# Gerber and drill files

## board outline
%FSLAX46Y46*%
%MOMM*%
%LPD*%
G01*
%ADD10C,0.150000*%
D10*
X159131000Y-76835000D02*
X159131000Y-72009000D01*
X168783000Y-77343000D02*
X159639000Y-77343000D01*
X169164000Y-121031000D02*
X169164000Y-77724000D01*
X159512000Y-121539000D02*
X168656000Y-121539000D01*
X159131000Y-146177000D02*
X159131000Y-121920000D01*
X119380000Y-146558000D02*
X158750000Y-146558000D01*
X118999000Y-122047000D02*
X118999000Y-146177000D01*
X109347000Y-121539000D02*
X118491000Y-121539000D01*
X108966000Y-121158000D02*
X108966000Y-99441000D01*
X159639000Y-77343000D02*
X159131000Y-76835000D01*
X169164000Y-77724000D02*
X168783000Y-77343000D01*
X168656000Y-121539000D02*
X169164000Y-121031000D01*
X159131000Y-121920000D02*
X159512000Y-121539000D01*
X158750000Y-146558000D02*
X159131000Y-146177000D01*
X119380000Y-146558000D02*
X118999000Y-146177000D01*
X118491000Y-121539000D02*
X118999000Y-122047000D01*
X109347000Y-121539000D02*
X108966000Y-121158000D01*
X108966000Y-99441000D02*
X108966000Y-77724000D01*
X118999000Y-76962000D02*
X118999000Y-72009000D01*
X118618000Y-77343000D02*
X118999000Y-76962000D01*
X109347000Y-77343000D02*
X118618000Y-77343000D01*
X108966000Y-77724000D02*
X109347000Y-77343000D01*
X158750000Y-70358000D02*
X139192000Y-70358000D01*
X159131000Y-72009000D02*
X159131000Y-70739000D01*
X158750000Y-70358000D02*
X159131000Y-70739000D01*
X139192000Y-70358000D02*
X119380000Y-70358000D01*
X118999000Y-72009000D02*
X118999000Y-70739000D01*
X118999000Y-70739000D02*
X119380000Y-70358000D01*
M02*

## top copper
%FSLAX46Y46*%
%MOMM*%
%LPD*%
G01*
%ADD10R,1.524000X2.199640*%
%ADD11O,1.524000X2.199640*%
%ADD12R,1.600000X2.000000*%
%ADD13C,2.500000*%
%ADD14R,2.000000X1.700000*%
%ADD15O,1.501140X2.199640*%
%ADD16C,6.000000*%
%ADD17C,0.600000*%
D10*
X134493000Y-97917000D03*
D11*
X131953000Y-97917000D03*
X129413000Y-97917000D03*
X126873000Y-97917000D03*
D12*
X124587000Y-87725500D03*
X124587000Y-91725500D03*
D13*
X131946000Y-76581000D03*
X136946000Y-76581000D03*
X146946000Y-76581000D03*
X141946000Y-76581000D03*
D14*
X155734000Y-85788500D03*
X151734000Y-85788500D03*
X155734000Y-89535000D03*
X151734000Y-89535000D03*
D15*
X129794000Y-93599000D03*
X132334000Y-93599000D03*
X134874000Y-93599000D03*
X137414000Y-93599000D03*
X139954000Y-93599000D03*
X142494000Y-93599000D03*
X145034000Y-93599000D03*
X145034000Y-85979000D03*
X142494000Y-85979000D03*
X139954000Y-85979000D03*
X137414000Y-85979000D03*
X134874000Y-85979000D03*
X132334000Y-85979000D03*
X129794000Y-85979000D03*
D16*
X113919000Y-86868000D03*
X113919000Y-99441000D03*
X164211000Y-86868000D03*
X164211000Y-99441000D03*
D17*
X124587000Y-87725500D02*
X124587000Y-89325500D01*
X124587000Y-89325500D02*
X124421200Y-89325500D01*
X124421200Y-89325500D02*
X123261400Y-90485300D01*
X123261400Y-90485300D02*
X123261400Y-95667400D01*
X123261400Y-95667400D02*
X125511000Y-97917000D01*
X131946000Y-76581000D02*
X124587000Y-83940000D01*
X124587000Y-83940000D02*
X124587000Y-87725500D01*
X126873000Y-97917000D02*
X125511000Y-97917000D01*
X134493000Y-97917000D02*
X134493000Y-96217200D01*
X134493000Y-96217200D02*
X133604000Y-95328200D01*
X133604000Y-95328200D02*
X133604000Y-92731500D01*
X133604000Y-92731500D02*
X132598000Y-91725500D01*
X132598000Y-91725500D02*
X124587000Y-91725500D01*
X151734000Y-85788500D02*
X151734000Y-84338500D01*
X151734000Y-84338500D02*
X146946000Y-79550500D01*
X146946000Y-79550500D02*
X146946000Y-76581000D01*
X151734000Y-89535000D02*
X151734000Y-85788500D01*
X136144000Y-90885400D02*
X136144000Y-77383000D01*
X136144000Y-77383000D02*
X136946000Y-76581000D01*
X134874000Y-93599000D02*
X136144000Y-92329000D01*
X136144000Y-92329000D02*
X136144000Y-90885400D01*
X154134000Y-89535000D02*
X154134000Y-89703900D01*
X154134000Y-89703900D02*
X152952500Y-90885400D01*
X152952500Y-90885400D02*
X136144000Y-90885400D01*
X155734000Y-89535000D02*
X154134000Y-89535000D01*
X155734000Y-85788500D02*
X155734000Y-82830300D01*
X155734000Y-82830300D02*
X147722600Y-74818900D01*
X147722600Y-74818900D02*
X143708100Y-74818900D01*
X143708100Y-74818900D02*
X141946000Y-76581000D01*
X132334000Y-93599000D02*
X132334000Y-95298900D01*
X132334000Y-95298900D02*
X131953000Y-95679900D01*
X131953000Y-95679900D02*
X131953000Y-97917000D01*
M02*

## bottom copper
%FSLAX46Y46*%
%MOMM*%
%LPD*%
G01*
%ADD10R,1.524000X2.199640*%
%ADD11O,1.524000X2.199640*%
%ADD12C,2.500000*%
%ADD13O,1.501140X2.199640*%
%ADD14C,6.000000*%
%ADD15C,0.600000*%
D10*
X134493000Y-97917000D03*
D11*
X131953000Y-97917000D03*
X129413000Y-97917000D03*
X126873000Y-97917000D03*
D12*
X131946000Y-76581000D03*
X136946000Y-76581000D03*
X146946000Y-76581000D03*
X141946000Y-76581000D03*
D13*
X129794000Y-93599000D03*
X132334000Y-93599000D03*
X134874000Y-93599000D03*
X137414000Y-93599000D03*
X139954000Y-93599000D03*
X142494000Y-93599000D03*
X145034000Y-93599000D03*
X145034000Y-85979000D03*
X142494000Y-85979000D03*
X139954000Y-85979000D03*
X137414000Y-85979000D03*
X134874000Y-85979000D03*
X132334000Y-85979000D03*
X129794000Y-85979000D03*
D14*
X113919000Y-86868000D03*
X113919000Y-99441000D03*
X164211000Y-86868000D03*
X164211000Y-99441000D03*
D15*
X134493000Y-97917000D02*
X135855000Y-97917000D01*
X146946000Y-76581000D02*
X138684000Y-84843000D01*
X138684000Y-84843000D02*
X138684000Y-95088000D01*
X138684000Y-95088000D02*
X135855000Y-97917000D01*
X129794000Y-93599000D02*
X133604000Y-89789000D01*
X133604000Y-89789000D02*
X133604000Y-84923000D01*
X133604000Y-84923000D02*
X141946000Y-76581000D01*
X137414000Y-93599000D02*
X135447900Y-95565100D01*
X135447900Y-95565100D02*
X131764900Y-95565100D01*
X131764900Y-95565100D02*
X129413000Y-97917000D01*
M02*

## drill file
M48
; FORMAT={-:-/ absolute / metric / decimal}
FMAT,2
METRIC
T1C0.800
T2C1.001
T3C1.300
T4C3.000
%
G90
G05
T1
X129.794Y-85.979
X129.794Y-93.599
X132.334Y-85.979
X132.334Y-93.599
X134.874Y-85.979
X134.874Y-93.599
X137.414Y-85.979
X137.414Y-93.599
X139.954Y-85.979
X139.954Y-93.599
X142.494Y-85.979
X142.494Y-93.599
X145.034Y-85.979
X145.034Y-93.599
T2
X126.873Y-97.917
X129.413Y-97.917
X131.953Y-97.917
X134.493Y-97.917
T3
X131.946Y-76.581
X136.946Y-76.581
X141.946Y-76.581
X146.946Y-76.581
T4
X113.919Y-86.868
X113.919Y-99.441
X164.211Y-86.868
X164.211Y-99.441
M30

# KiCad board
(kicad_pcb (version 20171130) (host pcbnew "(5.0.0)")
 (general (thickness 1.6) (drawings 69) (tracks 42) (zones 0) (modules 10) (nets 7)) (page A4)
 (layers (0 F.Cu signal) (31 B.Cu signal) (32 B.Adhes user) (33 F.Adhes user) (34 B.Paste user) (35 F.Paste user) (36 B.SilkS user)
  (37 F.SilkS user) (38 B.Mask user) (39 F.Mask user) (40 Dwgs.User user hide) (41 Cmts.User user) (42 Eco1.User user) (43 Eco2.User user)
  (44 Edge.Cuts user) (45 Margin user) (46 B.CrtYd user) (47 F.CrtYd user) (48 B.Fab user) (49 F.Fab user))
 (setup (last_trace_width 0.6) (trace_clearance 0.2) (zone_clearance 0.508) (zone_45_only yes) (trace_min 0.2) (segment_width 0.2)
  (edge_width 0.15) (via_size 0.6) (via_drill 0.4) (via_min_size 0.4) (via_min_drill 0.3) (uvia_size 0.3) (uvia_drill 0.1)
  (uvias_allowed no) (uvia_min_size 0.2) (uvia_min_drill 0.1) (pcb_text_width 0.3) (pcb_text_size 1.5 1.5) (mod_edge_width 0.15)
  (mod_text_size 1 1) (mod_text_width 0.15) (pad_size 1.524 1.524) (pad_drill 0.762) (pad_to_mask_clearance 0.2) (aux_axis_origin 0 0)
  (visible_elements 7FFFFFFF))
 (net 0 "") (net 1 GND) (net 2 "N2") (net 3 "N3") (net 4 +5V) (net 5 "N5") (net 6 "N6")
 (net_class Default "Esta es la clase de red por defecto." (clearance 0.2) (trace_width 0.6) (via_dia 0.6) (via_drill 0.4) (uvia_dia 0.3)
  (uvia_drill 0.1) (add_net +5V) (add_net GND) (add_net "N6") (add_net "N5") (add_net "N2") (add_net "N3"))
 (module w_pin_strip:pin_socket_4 (layer F.Cu) (at 130.683 97.917 180)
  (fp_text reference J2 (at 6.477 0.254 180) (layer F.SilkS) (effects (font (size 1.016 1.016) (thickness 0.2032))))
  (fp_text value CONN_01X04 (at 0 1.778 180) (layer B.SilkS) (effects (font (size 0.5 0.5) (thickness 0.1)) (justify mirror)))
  (pad 1 thru_hole rect (at -3.81 0 180) (size 1.524 2.19964) (drill 1.00076) (layers *.Cu *.Mask F.SilkS) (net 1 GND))
  (pad 2 thru_hole oval (at -1.27 0 180) (size 1.524 2.19964) (drill 1.00076) (layers *.Cu *.Mask F.SilkS) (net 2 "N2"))
  (pad 3 thru_hole oval (at 1.27 0 180) (size 1.524 2.19964) (drill 1.00076) (layers *.Cu *.Mask F.SilkS) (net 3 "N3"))
  (pad 4 thru_hole oval (at 3.81 0 180) (size 1.524 2.19964) (drill 1.00076) (layers *.Cu *.Mask F.SilkS) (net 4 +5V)))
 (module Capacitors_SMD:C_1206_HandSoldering (layer F.Cu) (at 124.587 89.7255 270)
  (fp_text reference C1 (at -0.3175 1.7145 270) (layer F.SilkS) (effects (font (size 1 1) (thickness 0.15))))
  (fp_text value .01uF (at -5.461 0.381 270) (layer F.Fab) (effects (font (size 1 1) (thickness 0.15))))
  (pad 1 smd rect (at -2 0 270) (size 2 1.6) (layers F.Cu F.Paste F.Mask) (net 4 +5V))
  (pad 2 smd rect (at 2 0 270) (size 2 1.6) (layers F.Cu F.Paste F.Mask) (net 1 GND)))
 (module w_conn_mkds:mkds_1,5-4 (layer F.Cu) (at 139.446 76.581 180)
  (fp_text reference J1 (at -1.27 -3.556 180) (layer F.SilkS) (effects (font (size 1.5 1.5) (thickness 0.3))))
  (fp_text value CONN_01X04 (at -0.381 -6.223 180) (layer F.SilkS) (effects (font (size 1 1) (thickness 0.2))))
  (pad 4 thru_hole circle (at 7.5 0 180) (size 2.5 2.5) (drill 1.3) (layers *.Cu *.Mask F.SilkS) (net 4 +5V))
  (pad 3 thru_hole circle (at 2.5 0 180) (size 2.5 2.5) (drill 1.3) (layers *.Cu *.Mask F.SilkS) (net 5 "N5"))
  (pad 1 thru_hole circle (at -7.5 0 180) (size 2.5 2.5) (drill 1.3) (layers *.Cu *.Mask F.SilkS) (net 1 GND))
  (pad 2 thru_hole circle (at -2.5 0 180) (size 2.5 2.5) (drill 1.3) (layers *.Cu *.Mask F.SilkS) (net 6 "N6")))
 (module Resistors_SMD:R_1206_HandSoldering (layer F.Cu) (at 153.734 85.7885 180)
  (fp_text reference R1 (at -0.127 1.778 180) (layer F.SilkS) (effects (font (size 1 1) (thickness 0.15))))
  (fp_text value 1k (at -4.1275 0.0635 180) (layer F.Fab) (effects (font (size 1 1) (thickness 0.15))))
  (pad 1 smd rect (at -2 0 180) (size 2 1.7) (layers F.Cu F.Paste F.Mask) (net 6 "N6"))
  (pad 2 smd rect (at 2 0 180) (size 2 1.7) (layers F.Cu F.Paste F.Mask) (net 1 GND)))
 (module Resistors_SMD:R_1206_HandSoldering (layer F.Cu) (at 153.734 89.535 180)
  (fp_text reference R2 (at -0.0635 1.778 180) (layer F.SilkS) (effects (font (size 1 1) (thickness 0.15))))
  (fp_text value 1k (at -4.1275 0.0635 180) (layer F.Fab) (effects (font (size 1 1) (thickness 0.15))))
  (pad 1 smd rect (at -2 0 180) (size 2 1.7) (layers F.Cu F.Paste F.Mask) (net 5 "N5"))
  (pad 2 smd rect (at 2 0 180) (size 2 1.7) (layers F.Cu F.Paste F.Mask) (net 1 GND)))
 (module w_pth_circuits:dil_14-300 (layer F.Cu) (at 137.414 89.789)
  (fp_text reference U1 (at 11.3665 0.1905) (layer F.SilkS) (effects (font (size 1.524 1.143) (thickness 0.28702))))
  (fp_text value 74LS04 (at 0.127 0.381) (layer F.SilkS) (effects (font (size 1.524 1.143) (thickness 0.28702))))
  (pad 1 thru_hole oval (at -7.62 3.81) (size 1.50114 2.19964) (drill 0.8001) (layers *.Cu *.Mask F.SilkS) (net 6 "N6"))
  (pad 2 thru_hole oval (at -5.08 3.81) (size 1.50114 2.19964) (drill 0.8001) (layers *.Cu *.Mask F.SilkS) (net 2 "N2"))
  (pad 3 thru_hole oval (at -2.54 3.81) (size 1.50114 2.19964) (drill 0.8001) (layers *.Cu *.Mask F.SilkS) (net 5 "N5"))
  (pad 4 thru_hole oval (at 0 3.81) (size 1.50114 2.19964) (drill 0.8001) (layers *.Cu *.Mask F.SilkS) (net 3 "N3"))
  (pad 5 thru_hole oval (at 2.54 3.81) (size 1.50114 2.19964) (drill 0.8001) (layers *.Cu *.Mask F.SilkS))
  (pad 6 thru_hole oval (at 5.08 3.81) (size 1.50114 2.19964) (drill 0.8001) (layers *.Cu *.Mask F.SilkS))
  (pad 7 thru_hole oval (at 7.62 3.81) (size 1.50114 2.19964) (drill 0.8001) (layers *.Cu *.Mask F.SilkS))
  (pad 8 thru_hole oval (at 7.62 -3.81) (size 1.50114 2.19964) (drill 0.8001) (layers *.Cu *.Mask F.SilkS))
  (pad 9 thru_hole oval (at 5.08 -3.81) (size 1.50114 2.19964) (drill 0.8001) (layers *.Cu *.Mask F.SilkS))
  (pad 10 thru_hole oval (at 2.54 -3.81) (size 1.50114 2.19964) (drill 0.8001) (layers *.Cu *.Mask F.SilkS))
  (pad 11 thru_hole oval (at 0 -3.81) (size 1.50114 2.19964) (drill 0.8001) (layers *.Cu *.Mask F.SilkS))
  (pad 12 thru_hole oval (at -2.54 -3.81) (size 1.50114 2.19964) (drill 0.8001) (layers *.Cu *.Mask F.SilkS))
  (pad 13 thru_hole oval (at -5.08 -3.81) (size 1.50114 2.19964) (drill 0.8001) (layers *.Cu *.Mask F.SilkS))
  (pad 14 thru_hole oval (at -7.62 -3.81) (size 1.50114 2.19964) (drill 0.8001) (layers *.Cu *.Mask F.SilkS)))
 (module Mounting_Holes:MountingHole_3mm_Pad (layer F.Cu) (at 113.919 86.868)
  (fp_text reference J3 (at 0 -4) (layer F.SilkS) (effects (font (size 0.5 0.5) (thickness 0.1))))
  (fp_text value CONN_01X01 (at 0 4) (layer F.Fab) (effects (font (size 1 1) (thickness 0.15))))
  (pad 1 thru_hole circle (at 0 0) (size 6 6) (drill 3) (layers *.Cu *.Mask)))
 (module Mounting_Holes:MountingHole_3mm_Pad (layer F.Cu) (at 113.919 99.441)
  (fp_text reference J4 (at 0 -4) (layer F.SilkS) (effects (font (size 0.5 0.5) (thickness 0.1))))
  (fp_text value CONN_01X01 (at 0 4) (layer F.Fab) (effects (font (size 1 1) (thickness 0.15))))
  (pad 1 thru_hole circle (at 0 0) (size 6 6) (drill 3) (layers *.Cu *.Mask)))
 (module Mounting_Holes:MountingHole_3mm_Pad (layer F.Cu) (at 164.211 86.868)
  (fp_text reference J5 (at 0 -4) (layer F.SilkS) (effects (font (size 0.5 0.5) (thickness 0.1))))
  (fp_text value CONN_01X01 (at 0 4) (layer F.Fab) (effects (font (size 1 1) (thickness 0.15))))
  (pad 1 thru_hole circle (at 0 0) (size 6 6) (drill 3) (layers *.Cu *.Mask)))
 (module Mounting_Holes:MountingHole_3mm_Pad (layer F.Cu) (at 164.211 99.441)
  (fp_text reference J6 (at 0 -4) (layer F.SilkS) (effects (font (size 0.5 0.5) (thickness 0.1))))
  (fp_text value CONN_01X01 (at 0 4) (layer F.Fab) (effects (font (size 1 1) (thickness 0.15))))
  (pad 1 thru_hole circle (at 0 0) (size 6 6) (drill 3) (layers *.Cu *.Mask)))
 (gr_line (start 159.131 76.835) (end 159.131 72.009) (angle 90) (layer Edge.Cuts) (width 0.15))
 (gr_line (start 168.783 77.343) (end 159.639 77.343) (angle 90) (layer Edge.Cuts) (width 0.15))
 (gr_line (start 169.164 121.031) (end 169.164 77.724) (angle 90) (layer Edge.Cuts) (width 0.15))
 (gr_line (start 159.512 121.539) (end 168.656 121.539) (angle 90) (layer Edge.Cuts) (width 0.15))
 (gr_line (start 159.131 146.177) (end 159.131 121.92) (angle 90) (layer Edge.Cuts) (width 0.15))
 (gr_line (start 119.38 146.558) (end 158.75 146.558) (angle 90) (layer Edge.Cuts) (width 0.15))
 (gr_line (start 118.999 122.047) (end 118.999 146.177) (angle 90) (layer Edge.Cuts) (width 0.15))
 (gr_line (start 109.347 121.539) (end 118.491 121.539) (angle 90) (layer Edge.Cuts) (width 0.15))
 (gr_line (start 108.966 121.158) (end 108.966 99.441) (angle 90) (layer Edge.Cuts) (width 0.15))
 (gr_line (start 159.639 77.343) (end 159.131 76.835) (angle 90) (layer Edge.Cuts) (width 0.15))
 (gr_line (start 169.164 77.724) (end 168.783 77.343) (angle 90) (layer Edge.Cuts) (width 0.15))
 (gr_line (start 168.656 121.539) (end 169.164 121.031) (angle 90) (layer Edge.Cuts) (width 0.15))
 (gr_line (start 159.131 121.92) (end 159.512 121.539) (angle 90) (layer Edge.Cuts) (width 0.15))
 (gr_line (start 158.75 146.558) (end 159.131 146.177) (angle 90) (layer Edge.Cuts) (width 0.15))
 (gr_line (start 119.38 146.558) (end 118.999 146.177) (angle 90) (layer Edge.Cuts) (width 0.15))
 (gr_line (start 118.491 121.539) (end 118.999 122.047) (angle 90) (layer Edge.Cuts) (width 0.15))
 (gr_line (start 109.347 121.539) (end 108.966 121.158) (angle 90) (layer Edge.Cuts) (width 0.15))
 (gr_line (start 108.966 99.441) (end 108.966 77.724) (angle 90) (layer Edge.Cuts) (width 0.15))
 (gr_line (start 118.999 76.962) (end 118.999 72.009) (angle 90) (layer Edge.Cuts) (width 0.15))
 (gr_line (start 118.618 77.343) (end 118.999 76.962) (angle 90) (layer Edge.Cuts) (width 0.15))
 (gr_line (start 109.347 77.343) (end 118.618 77.343) (angle 90) (layer Edge.Cuts) (width 0.15))
 (gr_line (start 108.966 77.724) (end 109.347 77.343) (angle 90) (layer Edge.Cuts) (width 0.15))
 (gr_line (start 158.75 70.358) (end 139.192 70.358) (angle 90) (layer Edge.Cuts) (width 0.15))
 (gr_line (start 159.131 72.009) (end 159.131 70.739) (angle 90) (layer Edge.Cuts) (width 0.15))
 (gr_line (start 158.75 70.358) (end 159.131 70.739) (angle 90) (layer Edge.Cuts) (width 0.15))
 (gr_line (start 139.192 70.358) (end 119.38 70.358) (angle 90) (layer Edge.Cuts) (width 0.15))
 (gr_line (start 118.999 72.009) (end 118.999 70.739) (angle 90) (layer Edge.Cuts) (width 0.15))
 (gr_line (start 118.999 70.739) (end 119.38 70.358) (angle 90) (layer Edge.Cuts) (width 0.15))
 (segment (start 124.587 87.7255) (end 124.587 89.3255) (width 0.6) (layer F.Cu) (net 4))
 (segment (start 124.587 89.3255) (end 124.4212 89.3255) (width 0.6) (layer F.Cu) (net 4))
 (segment (start 124.4212 89.3255) (end 123.2614 90.4853) (width 0.6) (layer F.Cu) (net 4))
 (segment (start 123.2614 90.4853) (end 123.2614 95.6674) (width 0.6) (layer F.Cu) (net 4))
 (segment (start 123.2614 95.6674) (end 125.511 97.917) (width 0.6) (layer F.Cu) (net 4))
 (segment (start 131.946 76.581) (end 124.587 83.94) (width 0.6) (layer F.Cu) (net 4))
 (segment (start 124.587 83.94) (end 124.587 87.7255) (width 0.6) (layer F.Cu) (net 4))
 (segment (start 126.873 97.917) (end 125.511 97.917) (width 0.6) (layer F.Cu) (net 4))
 (segment (start 134.493 97.917) (end 134.493 96.2172) (width 0.6) (layer F.Cu) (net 1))
 (segment (start 134.493 96.2172) (end 133.604 95.3282) (width 0.6) (layer F.Cu) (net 1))
 (segment (start 133.604 95.3282) (end 133.604 92.7315) (width 0.6) (layer F.Cu) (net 1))
 (segment (start 133.604 92.7315) (end 132.598 91.7255) (width 0.6) (layer F.Cu) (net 1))
 (segment (start 132.598 91.7255) (end 124.587 91.7255) (width 0.6) (layer F.Cu) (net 1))
 (segment (start 134.493 97.917) (end 135.855 97.917) (width 0.6) (layer B.Cu) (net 1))
 (segment (start 146.946 76.581) (end 138.684 84.843) (width 0.6) (layer B.Cu) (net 1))
 (segment (start 138.684 84.843) (end 138.684 95.088) (width 0.6) (layer B.Cu) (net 1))
 (segment (start 138.684 95.088) (end 135.855 97.917) (width 0.6) (layer B.Cu) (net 1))
 (segment (start 151.734 85.7885) (end 151.734 84.3385) (width 0.6) (layer F.Cu) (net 1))
 (segment (start 151.734 84.3385) (end 146.946 79.5505) (width 0.6) (layer F.Cu) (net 1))
 (segment (start 146.946 79.5505) (end 146.946 76.581) (width 0.6) (layer F.Cu) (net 1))
 (segment (start 151.734 89.535) (end 151.734 85.7885) (width 0.6) (layer F.Cu) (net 1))
 (segment (start 136.144 90.8854) (end 136.144 77.383) (width 0.6) (layer F.Cu) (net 5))
 (segment (start 136.144 77.383) (end 136.946 76.581) (width 0.6) (layer F.Cu) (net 5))
 (segment (start 134.874 93.599) (end 136.144 92.329) (width 0.6) (layer F.Cu) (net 5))
 (segment (start 136.144 92.329) (end 136.144 90.8854) (width 0.6) (layer F.Cu) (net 5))
 (segment (start 154.134 89.535) (end 154.134 89.7039) (width 0.6) (layer F.Cu) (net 5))
 (segment (start 154.134 89.7039) (end 152.9525 90.8854) (width 0.6) (layer F.Cu) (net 5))
 (segment (start 152.9525 90.8854) (end 136.144 90.8854) (width 0.6) (layer F.Cu) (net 5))
 (segment (start 155.734 89.535) (end 154.134 89.535) (width 0.6) (layer F.Cu) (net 5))
 (segment (start 155.734 85.7885) (end 155.734 82.8303) (width 0.6) (layer F.Cu) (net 6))
 (segment (start 155.734 82.8303) (end 147.7226 74.8189) (width 0.6) (layer F.Cu) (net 6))
 (segment (start 147.7226 74.8189) (end 143.7081 74.8189) (width 0.6) (layer F.Cu) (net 6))
 (segment (start 143.7081 74.8189) (end 141.946 76.581) (width 0.6) (layer F.Cu) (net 6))
 (segment (start 129.794 93.599) (end 133.604 89.789) (width 0.6) (layer B.Cu) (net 6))
 (segment (start 133.604 89.789) (end 133.604 84.923) (width 0.6) (layer B.Cu) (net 6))
 (segment (start 133.604 84.923) (end 141.946 76.581) (width 0.6) (layer B.Cu) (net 6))
 (segment (start 132.334 93.599) (end 132.334 95.2989) (width 0.6) (layer F.Cu) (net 2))
 (segment (start 132.334 95.2989) (end 131.953 95.6799) (width 0.6) (layer F.Cu) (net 2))
 (segment (start 131.953 95.6799) (end 131.953 97.917) (width 0.6) (layer F.Cu) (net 2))
 (segment (start 137.414 93.599) (end 135.4479 95.5651) (width 0.6) (layer B.Cu) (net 3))
 (segment (start 135.4479 95.5651) (end 131.7649 95.5651) (width 0.6) (layer B.Cu) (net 3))
 (segment (start 131.7649 95.5651) (end 129.413 97.917) (width 0.6) (layer B.Cu) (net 3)))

